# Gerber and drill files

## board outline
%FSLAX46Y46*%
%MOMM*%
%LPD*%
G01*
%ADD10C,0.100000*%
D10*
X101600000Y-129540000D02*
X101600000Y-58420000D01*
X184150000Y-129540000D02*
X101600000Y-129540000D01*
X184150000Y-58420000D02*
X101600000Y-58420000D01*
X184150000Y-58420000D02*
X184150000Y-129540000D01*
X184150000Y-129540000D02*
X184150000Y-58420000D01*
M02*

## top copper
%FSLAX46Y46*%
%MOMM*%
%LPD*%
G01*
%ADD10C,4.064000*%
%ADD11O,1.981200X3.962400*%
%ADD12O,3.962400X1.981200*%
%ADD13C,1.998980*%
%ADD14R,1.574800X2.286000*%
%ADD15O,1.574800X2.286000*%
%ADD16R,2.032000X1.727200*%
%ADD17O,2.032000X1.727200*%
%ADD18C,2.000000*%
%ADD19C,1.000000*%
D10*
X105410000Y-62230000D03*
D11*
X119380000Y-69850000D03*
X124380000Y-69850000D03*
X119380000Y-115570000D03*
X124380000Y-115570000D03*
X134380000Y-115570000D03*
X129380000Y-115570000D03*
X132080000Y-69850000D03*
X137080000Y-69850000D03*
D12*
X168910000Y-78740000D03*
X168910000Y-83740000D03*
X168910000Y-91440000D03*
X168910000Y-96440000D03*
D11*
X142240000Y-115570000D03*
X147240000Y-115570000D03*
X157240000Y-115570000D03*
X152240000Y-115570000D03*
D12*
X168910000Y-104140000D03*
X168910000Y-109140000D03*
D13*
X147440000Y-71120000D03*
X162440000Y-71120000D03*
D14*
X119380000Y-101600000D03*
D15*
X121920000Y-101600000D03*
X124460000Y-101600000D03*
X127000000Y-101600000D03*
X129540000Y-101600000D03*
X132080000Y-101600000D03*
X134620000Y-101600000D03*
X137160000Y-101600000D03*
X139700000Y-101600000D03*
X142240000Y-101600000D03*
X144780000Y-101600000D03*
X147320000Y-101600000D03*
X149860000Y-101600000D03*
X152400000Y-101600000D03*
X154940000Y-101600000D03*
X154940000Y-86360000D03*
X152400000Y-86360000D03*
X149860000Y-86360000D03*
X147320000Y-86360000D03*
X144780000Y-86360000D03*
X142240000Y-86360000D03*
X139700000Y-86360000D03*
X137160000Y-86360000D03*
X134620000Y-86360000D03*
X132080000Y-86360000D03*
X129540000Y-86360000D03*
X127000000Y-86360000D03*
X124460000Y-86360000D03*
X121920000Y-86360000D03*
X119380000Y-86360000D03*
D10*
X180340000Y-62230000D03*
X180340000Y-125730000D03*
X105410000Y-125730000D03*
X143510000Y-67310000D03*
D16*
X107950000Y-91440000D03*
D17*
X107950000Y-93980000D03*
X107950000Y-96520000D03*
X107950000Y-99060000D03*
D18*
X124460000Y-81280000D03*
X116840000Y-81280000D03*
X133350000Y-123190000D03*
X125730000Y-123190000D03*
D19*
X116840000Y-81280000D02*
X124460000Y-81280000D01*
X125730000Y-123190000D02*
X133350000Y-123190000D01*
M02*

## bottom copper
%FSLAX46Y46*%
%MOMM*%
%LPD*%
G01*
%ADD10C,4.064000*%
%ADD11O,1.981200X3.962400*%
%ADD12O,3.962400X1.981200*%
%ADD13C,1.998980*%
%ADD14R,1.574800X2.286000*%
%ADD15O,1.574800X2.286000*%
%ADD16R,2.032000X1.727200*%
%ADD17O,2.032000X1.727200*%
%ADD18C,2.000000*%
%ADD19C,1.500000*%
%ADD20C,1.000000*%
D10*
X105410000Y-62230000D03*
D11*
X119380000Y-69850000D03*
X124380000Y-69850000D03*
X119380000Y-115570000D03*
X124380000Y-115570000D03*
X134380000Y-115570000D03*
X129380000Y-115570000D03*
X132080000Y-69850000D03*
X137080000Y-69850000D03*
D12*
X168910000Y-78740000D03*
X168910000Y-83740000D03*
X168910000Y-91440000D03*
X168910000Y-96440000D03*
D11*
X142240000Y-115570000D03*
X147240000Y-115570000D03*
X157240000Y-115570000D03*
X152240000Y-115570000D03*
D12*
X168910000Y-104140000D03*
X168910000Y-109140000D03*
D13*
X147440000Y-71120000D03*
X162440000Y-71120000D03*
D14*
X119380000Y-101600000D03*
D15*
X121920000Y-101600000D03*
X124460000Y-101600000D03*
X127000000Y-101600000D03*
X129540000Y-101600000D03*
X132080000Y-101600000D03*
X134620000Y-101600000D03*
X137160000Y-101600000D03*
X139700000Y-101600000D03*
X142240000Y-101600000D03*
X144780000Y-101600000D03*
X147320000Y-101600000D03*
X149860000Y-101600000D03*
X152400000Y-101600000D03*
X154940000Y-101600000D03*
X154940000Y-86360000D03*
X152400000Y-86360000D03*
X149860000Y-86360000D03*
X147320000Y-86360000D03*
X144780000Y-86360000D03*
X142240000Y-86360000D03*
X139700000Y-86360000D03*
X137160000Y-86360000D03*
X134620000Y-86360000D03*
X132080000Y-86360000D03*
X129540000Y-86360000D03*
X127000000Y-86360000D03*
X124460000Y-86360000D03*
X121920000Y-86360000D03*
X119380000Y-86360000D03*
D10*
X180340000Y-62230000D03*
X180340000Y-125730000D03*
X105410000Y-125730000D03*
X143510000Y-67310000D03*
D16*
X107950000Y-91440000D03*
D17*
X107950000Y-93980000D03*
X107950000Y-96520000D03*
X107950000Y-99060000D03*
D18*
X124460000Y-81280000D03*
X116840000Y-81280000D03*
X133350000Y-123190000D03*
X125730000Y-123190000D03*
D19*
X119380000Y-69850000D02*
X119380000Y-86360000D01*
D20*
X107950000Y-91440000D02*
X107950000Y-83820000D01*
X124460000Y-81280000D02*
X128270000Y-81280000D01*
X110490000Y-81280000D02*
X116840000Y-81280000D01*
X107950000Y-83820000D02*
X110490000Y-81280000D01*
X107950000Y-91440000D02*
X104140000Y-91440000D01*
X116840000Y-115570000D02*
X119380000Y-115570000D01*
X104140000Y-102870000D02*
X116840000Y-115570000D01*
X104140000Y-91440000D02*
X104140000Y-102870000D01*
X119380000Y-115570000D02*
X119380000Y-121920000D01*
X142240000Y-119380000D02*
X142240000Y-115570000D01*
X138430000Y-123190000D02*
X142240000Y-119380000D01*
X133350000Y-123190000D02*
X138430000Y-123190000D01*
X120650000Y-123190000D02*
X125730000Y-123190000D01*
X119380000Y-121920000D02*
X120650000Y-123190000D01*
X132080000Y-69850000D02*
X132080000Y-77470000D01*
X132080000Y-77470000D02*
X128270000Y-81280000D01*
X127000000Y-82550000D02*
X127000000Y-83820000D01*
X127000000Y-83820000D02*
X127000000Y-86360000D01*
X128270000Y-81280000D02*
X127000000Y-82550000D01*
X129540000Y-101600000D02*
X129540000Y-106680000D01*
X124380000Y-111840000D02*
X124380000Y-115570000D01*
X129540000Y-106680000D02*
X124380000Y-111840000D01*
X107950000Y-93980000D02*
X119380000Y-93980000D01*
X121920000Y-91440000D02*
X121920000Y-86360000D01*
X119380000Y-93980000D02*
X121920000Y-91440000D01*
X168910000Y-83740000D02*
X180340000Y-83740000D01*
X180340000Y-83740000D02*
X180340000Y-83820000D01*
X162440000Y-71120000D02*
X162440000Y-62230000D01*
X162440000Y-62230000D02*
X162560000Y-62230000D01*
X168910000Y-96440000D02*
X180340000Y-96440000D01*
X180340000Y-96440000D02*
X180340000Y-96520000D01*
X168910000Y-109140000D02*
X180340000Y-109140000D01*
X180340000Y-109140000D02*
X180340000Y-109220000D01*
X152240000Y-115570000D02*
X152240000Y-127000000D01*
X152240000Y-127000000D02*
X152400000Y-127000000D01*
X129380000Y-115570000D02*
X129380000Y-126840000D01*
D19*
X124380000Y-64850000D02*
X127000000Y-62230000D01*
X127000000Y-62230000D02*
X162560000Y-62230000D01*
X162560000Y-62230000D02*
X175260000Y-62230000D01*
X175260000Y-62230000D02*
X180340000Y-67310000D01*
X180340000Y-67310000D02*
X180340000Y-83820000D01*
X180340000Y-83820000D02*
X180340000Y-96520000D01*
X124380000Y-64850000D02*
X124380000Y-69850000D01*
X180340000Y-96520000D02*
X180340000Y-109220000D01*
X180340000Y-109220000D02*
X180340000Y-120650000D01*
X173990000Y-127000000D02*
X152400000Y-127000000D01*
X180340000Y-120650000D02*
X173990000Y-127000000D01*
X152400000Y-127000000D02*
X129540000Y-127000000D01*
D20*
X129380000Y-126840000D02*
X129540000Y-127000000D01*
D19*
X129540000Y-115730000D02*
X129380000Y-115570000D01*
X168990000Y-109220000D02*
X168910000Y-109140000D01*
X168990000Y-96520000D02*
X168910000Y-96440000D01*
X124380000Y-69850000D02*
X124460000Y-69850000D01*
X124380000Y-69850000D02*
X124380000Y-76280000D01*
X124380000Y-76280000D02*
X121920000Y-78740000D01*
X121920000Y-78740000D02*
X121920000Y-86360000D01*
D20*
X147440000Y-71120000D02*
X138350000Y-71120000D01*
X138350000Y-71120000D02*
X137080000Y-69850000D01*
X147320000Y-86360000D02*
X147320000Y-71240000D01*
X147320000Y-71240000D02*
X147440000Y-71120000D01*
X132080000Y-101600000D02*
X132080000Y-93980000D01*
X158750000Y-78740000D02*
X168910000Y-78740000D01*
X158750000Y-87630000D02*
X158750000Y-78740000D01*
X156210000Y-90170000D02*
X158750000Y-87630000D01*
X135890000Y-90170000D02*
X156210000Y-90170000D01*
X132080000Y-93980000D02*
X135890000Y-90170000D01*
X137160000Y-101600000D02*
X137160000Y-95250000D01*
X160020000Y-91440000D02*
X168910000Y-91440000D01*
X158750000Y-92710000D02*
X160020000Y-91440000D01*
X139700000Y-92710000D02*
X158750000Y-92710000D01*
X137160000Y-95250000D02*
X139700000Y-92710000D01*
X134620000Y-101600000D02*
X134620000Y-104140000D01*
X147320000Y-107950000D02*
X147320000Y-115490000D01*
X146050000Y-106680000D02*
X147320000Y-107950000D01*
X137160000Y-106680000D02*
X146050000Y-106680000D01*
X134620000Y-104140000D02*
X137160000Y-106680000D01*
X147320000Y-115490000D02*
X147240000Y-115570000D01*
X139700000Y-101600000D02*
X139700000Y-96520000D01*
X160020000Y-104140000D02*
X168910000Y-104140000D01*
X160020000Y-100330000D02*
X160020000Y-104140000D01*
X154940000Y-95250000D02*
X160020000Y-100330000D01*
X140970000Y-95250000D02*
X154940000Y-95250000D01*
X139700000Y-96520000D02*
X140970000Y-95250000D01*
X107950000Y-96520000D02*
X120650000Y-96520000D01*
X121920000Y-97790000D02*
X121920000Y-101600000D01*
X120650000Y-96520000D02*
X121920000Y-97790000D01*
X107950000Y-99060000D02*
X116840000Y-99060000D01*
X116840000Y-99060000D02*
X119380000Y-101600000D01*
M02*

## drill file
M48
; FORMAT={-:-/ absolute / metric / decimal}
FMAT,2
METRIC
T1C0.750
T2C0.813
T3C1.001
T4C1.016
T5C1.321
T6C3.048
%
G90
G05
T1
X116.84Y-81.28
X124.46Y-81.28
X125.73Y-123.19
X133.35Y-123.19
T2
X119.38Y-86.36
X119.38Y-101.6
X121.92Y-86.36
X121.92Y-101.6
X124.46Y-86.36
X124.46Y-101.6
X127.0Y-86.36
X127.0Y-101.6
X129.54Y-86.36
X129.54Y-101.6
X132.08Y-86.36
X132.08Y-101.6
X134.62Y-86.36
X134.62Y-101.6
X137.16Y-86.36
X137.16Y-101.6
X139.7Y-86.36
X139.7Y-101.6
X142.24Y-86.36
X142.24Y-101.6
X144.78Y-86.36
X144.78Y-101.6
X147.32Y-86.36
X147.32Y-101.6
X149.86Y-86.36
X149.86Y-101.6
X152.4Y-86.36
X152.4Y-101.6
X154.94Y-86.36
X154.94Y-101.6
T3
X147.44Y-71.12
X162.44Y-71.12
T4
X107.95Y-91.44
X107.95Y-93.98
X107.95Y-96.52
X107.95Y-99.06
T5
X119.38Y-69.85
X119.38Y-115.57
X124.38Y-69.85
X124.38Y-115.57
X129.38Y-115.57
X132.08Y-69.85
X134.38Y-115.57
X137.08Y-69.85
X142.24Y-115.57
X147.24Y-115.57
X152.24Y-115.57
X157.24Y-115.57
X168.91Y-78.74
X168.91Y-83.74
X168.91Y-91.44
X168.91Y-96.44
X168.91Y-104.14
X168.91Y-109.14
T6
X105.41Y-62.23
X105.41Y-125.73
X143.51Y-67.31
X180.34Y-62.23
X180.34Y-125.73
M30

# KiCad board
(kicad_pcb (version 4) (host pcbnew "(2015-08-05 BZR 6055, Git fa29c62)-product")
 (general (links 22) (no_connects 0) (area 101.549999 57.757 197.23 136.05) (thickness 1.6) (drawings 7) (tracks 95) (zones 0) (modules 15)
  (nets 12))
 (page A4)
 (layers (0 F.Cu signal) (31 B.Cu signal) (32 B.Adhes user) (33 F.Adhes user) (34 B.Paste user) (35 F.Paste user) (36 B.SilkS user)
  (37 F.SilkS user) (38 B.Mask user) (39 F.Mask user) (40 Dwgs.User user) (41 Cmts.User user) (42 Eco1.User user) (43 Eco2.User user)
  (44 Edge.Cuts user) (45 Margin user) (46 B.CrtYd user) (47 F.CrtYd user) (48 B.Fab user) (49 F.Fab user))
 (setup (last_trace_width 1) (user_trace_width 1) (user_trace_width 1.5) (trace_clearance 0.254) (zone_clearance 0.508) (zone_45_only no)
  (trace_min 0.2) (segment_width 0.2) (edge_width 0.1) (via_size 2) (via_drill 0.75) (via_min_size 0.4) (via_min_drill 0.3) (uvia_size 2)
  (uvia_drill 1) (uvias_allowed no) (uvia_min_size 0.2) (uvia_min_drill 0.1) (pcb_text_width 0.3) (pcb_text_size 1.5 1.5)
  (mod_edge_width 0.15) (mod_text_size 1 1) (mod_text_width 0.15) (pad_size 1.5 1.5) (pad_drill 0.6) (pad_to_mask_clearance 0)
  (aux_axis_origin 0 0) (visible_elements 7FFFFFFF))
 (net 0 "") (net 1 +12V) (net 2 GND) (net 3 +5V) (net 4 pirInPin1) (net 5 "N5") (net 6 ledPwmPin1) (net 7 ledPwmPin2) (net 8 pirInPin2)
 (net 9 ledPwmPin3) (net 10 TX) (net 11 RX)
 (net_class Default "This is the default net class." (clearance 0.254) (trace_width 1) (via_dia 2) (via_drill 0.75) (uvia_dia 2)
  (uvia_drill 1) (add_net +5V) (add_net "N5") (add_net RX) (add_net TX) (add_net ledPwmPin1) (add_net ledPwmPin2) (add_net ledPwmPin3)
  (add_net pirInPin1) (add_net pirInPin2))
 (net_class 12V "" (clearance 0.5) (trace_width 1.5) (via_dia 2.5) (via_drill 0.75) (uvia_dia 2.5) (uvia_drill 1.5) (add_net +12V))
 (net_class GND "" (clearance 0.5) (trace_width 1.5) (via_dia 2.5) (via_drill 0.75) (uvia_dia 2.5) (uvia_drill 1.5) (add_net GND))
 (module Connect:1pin (layer F.Cu) (at 105.41 62.23)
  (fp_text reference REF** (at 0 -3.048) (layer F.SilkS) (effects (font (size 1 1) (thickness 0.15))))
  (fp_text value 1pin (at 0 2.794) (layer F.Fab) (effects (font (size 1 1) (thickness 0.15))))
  (pad 1 thru_hole circle (at 0 0) (size 4.064 4.064) (drill 3.048) (layers *.Cu *.Mask F.SilkS)))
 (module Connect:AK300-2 (layer F.Cu) (at 119.38 69.85)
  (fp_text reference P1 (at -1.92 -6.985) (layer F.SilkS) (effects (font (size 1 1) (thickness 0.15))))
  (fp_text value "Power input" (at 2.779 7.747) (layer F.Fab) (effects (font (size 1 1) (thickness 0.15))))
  (pad 1 thru_hole oval (at 0 0) (size 1.9812 3.9624) (drill 1.3208) (layers *.Cu F.Paste F.SilkS F.Mask) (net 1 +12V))
  (pad 2 thru_hole oval (at 5 0) (size 1.9812 3.9624) (drill 1.3208) (layers *.Cu F.Paste F.SilkS F.Mask) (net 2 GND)))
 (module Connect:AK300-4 (layer F.Cu) (at 119.38 115.57)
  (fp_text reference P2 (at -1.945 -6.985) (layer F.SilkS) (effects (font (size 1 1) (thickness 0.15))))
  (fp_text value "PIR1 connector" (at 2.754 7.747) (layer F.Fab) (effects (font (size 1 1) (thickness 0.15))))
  (pad 1 thru_hole oval (at 0 0) (size 1.9812 3.9624) (drill 1.3208) (layers *.Cu F.Paste F.SilkS F.Mask) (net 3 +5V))
  (pad 2 thru_hole oval (at 5 0) (size 1.9812 3.9624) (drill 1.3208) (layers *.Cu F.Paste F.SilkS F.Mask) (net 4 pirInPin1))
  (pad 4 thru_hole oval (at 15 0) (size 1.9812 3.9624) (drill 1.3208) (layers *.Cu F.Paste F.SilkS F.Mask))
  (pad 3 thru_hole oval (at 10 0) (size 1.9812 3.9624) (drill 1.3208) (layers *.Cu *.Mask F.SilkS) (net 2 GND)))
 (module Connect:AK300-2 (layer F.Cu) (at 132.08 69.85)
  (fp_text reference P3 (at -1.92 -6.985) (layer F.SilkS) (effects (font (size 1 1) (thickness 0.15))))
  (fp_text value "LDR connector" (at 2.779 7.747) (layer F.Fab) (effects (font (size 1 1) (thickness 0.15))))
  (pad 1 thru_hole oval (at 0 0) (size 1.9812 3.9624) (drill 1.3208) (layers *.Cu F.Paste F.SilkS F.Mask) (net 3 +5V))
  (pad 2 thru_hole oval (at 5 0) (size 1.9812 3.9624) (drill 1.3208) (layers *.Cu F.Paste F.SilkS F.Mask) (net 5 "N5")))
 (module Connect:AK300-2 (layer F.Cu) (at 168.91 78.74 270)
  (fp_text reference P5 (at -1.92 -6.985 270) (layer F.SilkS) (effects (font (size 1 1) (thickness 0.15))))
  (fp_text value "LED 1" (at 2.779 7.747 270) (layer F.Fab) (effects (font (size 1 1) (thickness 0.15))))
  (pad 1 thru_hole oval (at 0 0 270) (size 1.9812 3.9624) (drill 1.3208) (layers *.Cu F.Paste F.SilkS F.Mask) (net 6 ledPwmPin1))
  (pad 2 thru_hole oval (at 5 0 270) (size 1.9812 3.9624) (drill 1.3208) (layers *.Cu F.Paste F.SilkS F.Mask) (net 2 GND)))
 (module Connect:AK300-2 (layer F.Cu) (at 168.91 91.44 270)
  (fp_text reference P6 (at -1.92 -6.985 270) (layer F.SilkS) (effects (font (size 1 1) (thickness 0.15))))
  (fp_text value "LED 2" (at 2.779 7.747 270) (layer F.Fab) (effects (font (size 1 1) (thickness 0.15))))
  (pad 1 thru_hole oval (at 0 0 270) (size 1.9812 3.9624) (drill 1.3208) (layers *.Cu F.Paste F.SilkS F.Mask) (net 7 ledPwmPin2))
  (pad 2 thru_hole oval (at 5 0 270) (size 1.9812 3.9624) (drill 1.3208) (layers *.Cu F.Paste F.SilkS F.Mask) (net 2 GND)))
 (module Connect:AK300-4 (layer F.Cu) (at 142.24 115.57)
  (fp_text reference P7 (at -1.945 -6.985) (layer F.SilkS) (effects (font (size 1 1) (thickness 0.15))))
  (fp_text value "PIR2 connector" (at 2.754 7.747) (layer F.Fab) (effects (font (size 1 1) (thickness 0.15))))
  (pad 1 thru_hole oval (at 0 0) (size 1.9812 3.9624) (drill 1.3208) (layers *.Cu F.Paste F.SilkS F.Mask) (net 3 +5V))
  (pad 2 thru_hole oval (at 5 0) (size 1.9812 3.9624) (drill 1.3208) (layers *.Cu F.Paste F.SilkS F.Mask) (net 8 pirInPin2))
  (pad 4 thru_hole oval (at 15 0) (size 1.9812 3.9624) (drill 1.3208) (layers *.Cu F.Paste F.SilkS F.Mask))
  (pad 3 thru_hole oval (at 10 0) (size 1.9812 3.9624) (drill 1.3208) (layers *.Cu *.Mask F.SilkS) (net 2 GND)))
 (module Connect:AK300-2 (layer F.Cu) (at 168.91 104.14 270)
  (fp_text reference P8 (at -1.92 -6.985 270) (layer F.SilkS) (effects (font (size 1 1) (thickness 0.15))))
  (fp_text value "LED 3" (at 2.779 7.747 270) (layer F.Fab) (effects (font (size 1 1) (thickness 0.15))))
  (pad 1 thru_hole oval (at 0 0 270) (size 1.9812 3.9624) (drill 1.3208) (layers *.Cu F.Paste F.SilkS F.Mask) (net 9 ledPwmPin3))
  (pad 2 thru_hole oval (at 5 0 270) (size 1.9812 3.9624) (drill 1.3208) (layers *.Cu F.Paste F.SilkS F.Mask) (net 2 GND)))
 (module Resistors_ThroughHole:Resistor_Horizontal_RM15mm (layer F.Cu) (at 154.94 71.12)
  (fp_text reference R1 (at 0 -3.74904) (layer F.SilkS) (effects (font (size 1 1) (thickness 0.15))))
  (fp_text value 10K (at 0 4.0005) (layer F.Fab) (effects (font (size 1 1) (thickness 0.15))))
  (pad 1 thru_hole circle (at -7.5 0) (size 1.99898 1.99898) (drill 1.00076) (layers *.Cu *.SilkS *.Mask) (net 5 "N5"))
  (pad 2 thru_hole circle (at 7.5 0) (size 1.99898 1.99898) (drill 1.00076) (layers *.Cu *.SilkS *.Mask) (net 2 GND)))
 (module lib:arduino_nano (layer F.Cu) (at 138.43 93.98)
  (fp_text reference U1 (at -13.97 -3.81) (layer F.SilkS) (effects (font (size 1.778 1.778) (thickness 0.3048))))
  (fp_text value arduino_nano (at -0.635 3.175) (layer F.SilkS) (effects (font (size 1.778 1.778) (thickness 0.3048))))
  (pad TX1 thru_hole rect (at -19.05 7.62) (size 1.5748 2.286) (drill 0.8128) (layers *.Cu *.Mask F.SilkS) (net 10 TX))
  (pad RX0 thru_hole oval (at -16.51 7.62) (size 1.5748 2.286) (drill 0.8128) (layers *.Cu *.Mask F.SilkS) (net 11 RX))
  (pad RST1 thru_hole oval (at -13.97 7.62) (size 1.5748 2.286) (drill 0.8128) (layers *.Cu *.Mask F.SilkS))
  (pad GND1 thru_hole oval (at -11.43 7.62) (size 1.5748 2.286) (drill 0.8128) (layers *.Cu *.Mask F.SilkS))
  (pad D2 thru_hole oval (at -8.89 7.62) (size 1.5748 2.286) (drill 0.8128) (layers *.Cu *.Mask F.SilkS) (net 4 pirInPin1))
  (pad D3 thru_hole oval (at -6.35 7.62) (size 1.5748 2.286) (drill 0.8128) (layers *.Cu *.Mask F.SilkS) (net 6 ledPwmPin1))
  (pad D4 thru_hole oval (at -3.81 7.62) (size 1.5748 2.286) (drill 0.8128) (layers *.Cu *.Mask F.SilkS) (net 8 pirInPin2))
  (pad D5 thru_hole oval (at -1.27 7.62) (size 1.5748 2.286) (drill 0.8128) (layers *.Cu *.Mask F.SilkS) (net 7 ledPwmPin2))
  (pad D6 thru_hole oval (at 1.27 7.62) (size 1.5748 2.286) (drill 0.8128) (layers *.Cu *.Mask F.SilkS) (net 9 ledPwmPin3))
  (pad D7 thru_hole oval (at 3.81 7.62) (size 1.5748 2.286) (drill 0.8128) (layers *.Cu *.Mask F.SilkS))
  (pad D8 thru_hole oval (at 6.35 7.62) (size 1.5748 2.286) (drill 0.8128) (layers *.Cu *.Mask F.SilkS))
  (pad D9 thru_hole oval (at 8.89 7.62) (size 1.5748 2.286) (drill 0.8128) (layers *.Cu *.Mask F.SilkS))
  (pad D10 thru_hole oval (at 11.43 7.62) (size 1.5748 2.286) (drill 0.8128) (layers *.Cu *.Mask F.SilkS))
  (pad D11 thru_hole oval (at 13.97 7.62) (size 1.5748 2.286) (drill 0.8128) (layers *.Cu *.Mask F.SilkS))
  (pad D12 thru_hole oval (at 16.51 7.62) (size 1.5748 2.286) (drill 0.8128) (layers *.Cu *.Mask F.SilkS))
  (pad D13 thru_hole oval (at 16.51 -7.62) (size 1.5748 2.286) (drill 0.8128) (layers *.Cu *.Mask F.SilkS))
  (pad 3V3 thru_hole oval (at 13.97 -7.62) (size 1.5748 2.286) (drill 0.8128) (layers *.Cu *.Mask F.SilkS))
  (pad REF thru_hole oval (at 11.43 -7.62) (size 1.5748 2.286) (drill 0.8128) (layers *.Cu *.Mask F.SilkS))
  (pad A0 thru_hole oval (at 8.89 -7.62) (size 1.5748 2.286) (drill 0.8128) (layers *.Cu *.Mask F.SilkS) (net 5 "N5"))
  (pad A1 thru_hole oval (at 6.35 -7.62) (size 1.5748 2.286) (drill 0.8128) (layers *.Cu *.Mask F.SilkS))
  (pad A2 thru_hole oval (at 3.81 -7.62) (size 1.5748 2.286) (drill 0.8128) (layers *.Cu *.Mask F.SilkS))
  (pad A3 thru_hole oval (at 1.27 -7.62) (size 1.5748 2.286) (drill 0.8128) (layers *.Cu *.Mask F.SilkS))
  (pad A4 thru_hole oval (at -1.27 -7.62) (size 1.5748 2.286) (drill 0.8128) (layers *.Cu *.Mask F.SilkS))
  (pad A5 thru_hole oval (at -3.81 -7.62) (size 1.5748 2.286) (drill 0.8128) (layers *.Cu *.Mask F.SilkS))
  (pad A6 thru_hole oval (at -6.35 -7.62) (size 1.5748 2.286) (drill 0.8128) (layers *.Cu *.Mask F.SilkS))
  (pad A7 thru_hole oval (at -8.89 -7.62) (size 1.5748 2.286) (drill 0.8128) (layers *.Cu *.Mask F.SilkS))
  (pad 5V thru_hole oval (at -11.43 -7.62) (size 1.5748 2.286) (drill 0.8128) (layers *.Cu *.Mask F.SilkS) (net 3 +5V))
  (pad RST thru_hole oval (at -13.97 -7.62) (size 1.5748 2.286) (drill 0.8128) (layers *.Cu *.Mask F.SilkS))
  (pad GND thru_hole oval (at -16.51 -7.62) (size 1.5748 2.286) (drill 0.8128) (layers *.Cu *.Mask F.SilkS) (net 2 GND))
  (pad VIN thru_hole oval (at -19.05 -7.62) (size 1.5748 2.286) (drill 0.8128) (layers *.Cu *.Mask F.SilkS) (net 1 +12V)))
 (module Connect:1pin (layer F.Cu) (at 180.34 62.23)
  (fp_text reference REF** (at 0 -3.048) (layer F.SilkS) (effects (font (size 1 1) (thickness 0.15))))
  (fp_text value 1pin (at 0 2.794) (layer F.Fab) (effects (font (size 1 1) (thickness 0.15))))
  (pad 1 thru_hole circle (at 0 0) (size 4.064 4.064) (drill 3.048) (layers *.Cu *.Mask F.SilkS)))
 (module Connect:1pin (layer F.Cu) (at 180.34 125.73)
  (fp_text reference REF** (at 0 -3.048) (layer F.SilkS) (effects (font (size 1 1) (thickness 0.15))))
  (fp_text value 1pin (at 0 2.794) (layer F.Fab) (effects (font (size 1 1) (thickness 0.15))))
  (pad 1 thru_hole circle (at 0 0) (size 4.064 4.064) (drill 3.048) (layers *.Cu *.Mask F.SilkS)))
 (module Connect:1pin (layer F.Cu) (at 105.41 125.73)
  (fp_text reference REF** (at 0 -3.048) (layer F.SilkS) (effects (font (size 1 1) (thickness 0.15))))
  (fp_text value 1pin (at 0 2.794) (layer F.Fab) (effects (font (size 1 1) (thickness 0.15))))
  (pad 1 thru_hole circle (at 0 0) (size 4.064 4.064) (drill 3.048) (layers *.Cu *.Mask F.SilkS)))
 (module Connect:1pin (layer F.Cu) (at 143.51 67.31)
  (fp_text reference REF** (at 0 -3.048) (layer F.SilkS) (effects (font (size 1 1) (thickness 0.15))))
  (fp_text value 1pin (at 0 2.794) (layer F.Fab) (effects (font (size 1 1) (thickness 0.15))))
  (pad 1 thru_hole circle (at 0 0) (size 4.064 4.064) (drill 3.048) (layers *.Cu *.Mask F.SilkS)))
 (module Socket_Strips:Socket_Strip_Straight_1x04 (layer F.Cu) (at 107.95 91.44 270)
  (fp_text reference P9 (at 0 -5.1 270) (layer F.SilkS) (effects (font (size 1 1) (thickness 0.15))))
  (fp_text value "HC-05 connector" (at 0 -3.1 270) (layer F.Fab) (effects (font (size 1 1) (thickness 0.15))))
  (pad 1 thru_hole rect (at 0 0 270) (size 1.7272 2.032) (drill 1.016) (layers *.Cu *.Mask F.SilkS) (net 3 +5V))
  (pad 2 thru_hole oval (at 2.54 0 270) (size 1.7272 2.032) (drill 1.016) (layers *.Cu *.Mask F.SilkS) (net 2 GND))
  (pad 3 thru_hole oval (at 5.08 0 270) (size 1.7272 2.032) (drill 1.016) (layers *.Cu *.Mask F.SilkS) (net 11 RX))
  (pad 4 thru_hole oval (at 7.62 0 270) (size 1.7272 2.032) (drill 1.016) (layers *.Cu *.Mask F.SilkS) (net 10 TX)))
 (gr_line (start 101.6 129.54) (end 101.6 58.42) (angle 90) (layer Edge.Cuts) (width 0.1))
 (gr_line (start 184.15 129.54) (end 101.6 129.54) (angle 90) (layer Edge.Cuts) (width 0.1))
 (gr_line (start 184.15 58.42) (end 101.6 58.42) (angle 90) (layer Edge.Cuts) (width 0.1))
 (gr_line (start 184.15 58.42) (end 184.15 129.54) (angle 90) (layer Edge.Cuts) (width 0.1))
 (gr_line (start 184.15 129.54) (end 184.15 58.42) (angle 90) (layer Edge.Cuts) (width 0.1))
 (segment (start 119.38 69.85) (end 119.38 86.36) (width 1.5) (layer B.Cu) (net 1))
 (segment (start 107.95 91.44) (end 107.95 83.82) (width 1) (layer B.Cu) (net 3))
 (segment (start 124.46 81.28) (end 128.27 81.28) (width 1) (layer B.Cu) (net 3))
 (via (at 124.46 81.28) (size 2) (drill 0.75) (layers F.Cu B.Cu) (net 3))
 (segment (start 116.84 81.28) (end 124.46 81.28) (width 1) (layer F.Cu) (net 3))
 (via (at 116.84 81.28) (size 2) (drill 0.75) (layers F.Cu B.Cu) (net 3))
 (segment (start 110.49 81.28) (end 116.84 81.28) (width 1) (layer B.Cu) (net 3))
 (segment (start 107.95 83.82) (end 110.49 81.28) (width 1) (layer B.Cu) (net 3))
 (segment (start 107.95 91.44) (end 104.14 91.44) (width 1) (layer B.Cu) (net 3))
 (segment (start 116.84 115.57) (end 119.38 115.57) (width 1) (layer B.Cu) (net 3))
 (segment (start 104.14 102.87) (end 116.84 115.57) (width 1) (layer B.Cu) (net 3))
 (segment (start 104.14 91.44) (end 104.14 102.87) (width 1) (layer B.Cu) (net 3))
 (segment (start 119.38 115.57) (end 119.38 121.92) (width 1) (layer B.Cu) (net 3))
 (segment (start 142.24 119.38) (end 142.24 115.57) (width 1) (layer B.Cu) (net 3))
 (segment (start 138.43 123.19) (end 142.24 119.38) (width 1) (layer B.Cu) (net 3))
 (segment (start 133.35 123.19) (end 138.43 123.19) (width 1) (layer B.Cu) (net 3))
 (via (at 133.35 123.19) (size 2) (drill 0.75) (layers F.Cu B.Cu) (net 3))
 (segment (start 125.73 123.19) (end 133.35 123.19) (width 1) (layer F.Cu) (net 3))
 (via (at 125.73 123.19) (size 2) (drill 0.75) (layers F.Cu B.Cu) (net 3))
 (segment (start 120.65 123.19) (end 125.73 123.19) (width 1) (layer B.Cu) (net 3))
 (segment (start 119.38 121.92) (end 120.65 123.19) (width 1) (layer B.Cu) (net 3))
 (segment (start 132.08 69.85) (end 132.08 77.47) (width 1) (layer B.Cu) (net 3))
 (segment (start 132.08 77.47) (end 128.27 81.28) (width 1) (layer B.Cu) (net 3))
 (segment (start 127 82.55) (end 127 83.82) (width 1) (layer B.Cu) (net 3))
 (segment (start 127 83.82) (end 127 86.36) (width 1) (layer B.Cu) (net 3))
 (segment (start 128.27 81.28) (end 127 82.55) (width 1) (layer B.Cu) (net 3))
 (segment (start 129.54 101.6) (end 129.54 106.68) (width 1) (layer B.Cu) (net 4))
 (segment (start 124.38 111.84) (end 124.38 115.57) (width 1) (layer B.Cu) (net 4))
 (segment (start 129.54 106.68) (end 124.38 111.84) (width 1) (layer B.Cu) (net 4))
 (segment (start 107.95 93.98) (end 119.38 93.98) (width 1) (layer B.Cu) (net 2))
 (segment (start 121.92 91.44) (end 121.92 86.36) (width 1) (layer B.Cu) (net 2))
 (segment (start 119.38 93.98) (end 121.92 91.44) (width 1) (layer B.Cu) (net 2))
 (segment (start 168.91 83.74) (end 180.34 83.74) (width 1) (layer B.Cu) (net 2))
 (segment (start 180.34 83.74) (end 180.34 83.82) (width 1) (layer B.Cu) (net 2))
 (segment (start 162.44 71.12) (end 162.44 62.23) (width 1) (layer B.Cu) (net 2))
 (segment (start 162.44 62.23) (end 162.56 62.23) (width 1) (layer B.Cu) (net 2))
 (segment (start 168.91 96.44) (end 180.34 96.44) (width 1) (layer B.Cu) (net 2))
 (segment (start 180.34 96.44) (end 180.34 96.52) (width 1) (layer B.Cu) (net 2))
 (segment (start 168.91 109.14) (end 180.34 109.14) (width 1) (layer B.Cu) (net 2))
 (segment (start 180.34 109.14) (end 180.34 109.22) (width 1) (layer B.Cu) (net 2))
 (segment (start 152.24 115.57) (end 152.24 127) (width 1) (layer B.Cu) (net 2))
 (segment (start 152.24 127) (end 152.4 127) (width 1) (layer B.Cu) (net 2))
 (segment (start 129.38 115.57) (end 129.38 126.84) (width 1) (layer B.Cu) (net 2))
 (segment (start 124.38 64.85) (end 127 62.23) (width 1.5) (layer B.Cu) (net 2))
 (segment (start 127 62.23) (end 162.56 62.23) (width 1.5) (layer B.Cu) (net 2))
 (segment (start 162.56 62.23) (end 175.26 62.23) (width 1.5) (layer B.Cu) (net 2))
 (segment (start 175.26 62.23) (end 180.34 67.31) (width 1.5) (layer B.Cu) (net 2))
 (segment (start 180.34 67.31) (end 180.34 83.82) (width 1.5) (layer B.Cu) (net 2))
 (segment (start 180.34 83.82) (end 180.34 96.52) (width 1.5) (layer B.Cu) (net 2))
 (segment (start 124.38 64.85) (end 124.38 69.85) (width 1.5) (layer B.Cu) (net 2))
 (segment (start 180.34 96.52) (end 180.34 109.22) (width 1.5) (layer B.Cu) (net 2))
 (segment (start 180.34 109.22) (end 180.34 120.65) (width 1.5) (layer B.Cu) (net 2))
 (segment (start 173.99 127) (end 152.4 127) (width 1.5) (layer B.Cu) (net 2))
 (segment (start 180.34 120.65) (end 173.99 127) (width 1.5) (layer B.Cu) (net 2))
 (segment (start 152.4 127) (end 129.54 127) (width 1.5) (layer B.Cu) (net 2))
 (segment (start 129.38 126.84) (end 129.54 127) (width 1) (layer B.Cu) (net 2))
 (segment (start 129.54 115.73) (end 129.38 115.57) (width 1.5) (layer B.Cu) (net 2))
 (segment (start 168.99 109.22) (end 168.91 109.14) (width 1.5) (layer B.Cu) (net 2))
 (segment (start 168.99 96.52) (end 168.91 96.44) (width 1.5) (layer B.Cu) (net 2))
 (segment (start 124.38 69.85) (end 124.46 69.85) (width 1.5) (layer B.Cu) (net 2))
 (segment (start 124.38 69.85) (end 124.38 76.28) (width 1.5) (layer B.Cu) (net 2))
 (segment (start 124.38 76.28) (end 121.92 78.74) (width 1.5) (layer B.Cu) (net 2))
 (segment (start 121.92 78.74) (end 121.92 86.36) (width 1.5) (layer B.Cu) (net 2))
 (segment (start 147.44 71.12) (end 138.35 71.12) (width 1) (layer B.Cu) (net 5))
 (segment (start 138.35 71.12) (end 137.08 69.85) (width 1) (layer B.Cu) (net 5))
 (segment (start 147.32 86.36) (end 147.32 71.24) (width 1) (layer B.Cu) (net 5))
 (segment (start 147.32 71.24) (end 147.44 71.12) (width 1) (layer B.Cu) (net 5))
 (segment (start 132.08 101.6) (end 132.08 93.98) (width 1) (layer B.Cu) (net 6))
 (segment (start 158.75 78.74) (end 168.91 78.74) (width 1) (layer B.Cu) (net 6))
 (segment (start 158.75 87.63) (end 158.75 78.74) (width 1) (layer B.Cu) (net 6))
 (segment (start 156.21 90.17) (end 158.75 87.63) (width 1) (layer B.Cu) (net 6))
 (segment (start 135.89 90.17) (end 156.21 90.17) (width 1) (layer B.Cu) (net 6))
 (segment (start 132.08 93.98) (end 135.89 90.17) (width 1) (layer B.Cu) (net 6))
 (segment (start 137.16 101.6) (end 137.16 95.25) (width 1) (layer B.Cu) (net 7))
 (segment (start 160.02 91.44) (end 168.91 91.44) (width 1) (layer B.Cu) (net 7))
 (segment (start 158.75 92.71) (end 160.02 91.44) (width 1) (layer B.Cu) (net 7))
 (segment (start 139.7 92.71) (end 158.75 92.71) (width 1) (layer B.Cu) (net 7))
 (segment (start 137.16 95.25) (end 139.7 92.71) (width 1) (layer B.Cu) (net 7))
 (segment (start 134.62 101.6) (end 134.62 104.14) (width 1) (layer B.Cu) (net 8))
 (segment (start 147.32 107.95) (end 147.32 115.49) (width 1) (layer B.Cu) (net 8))
 (segment (start 146.05 106.68) (end 147.32 107.95) (width 1) (layer B.Cu) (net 8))
 (segment (start 137.16 106.68) (end 146.05 106.68) (width 1) (layer B.Cu) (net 8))
 (segment (start 134.62 104.14) (end 137.16 106.68) (width 1) (layer B.Cu) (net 8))
 (segment (start 147.32 115.49) (end 147.24 115.57) (width 1) (layer B.Cu) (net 8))
 (segment (start 139.7 101.6) (end 139.7 96.52) (width 1) (layer B.Cu) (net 9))
 (segment (start 160.02 104.14) (end 168.91 104.14) (width 1) (layer B.Cu) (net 9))
 (segment (start 160.02 100.33) (end 160.02 104.14) (width 1) (layer B.Cu) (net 9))
 (segment (start 154.94 95.25) (end 160.02 100.33) (width 1) (layer B.Cu) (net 9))
 (segment (start 140.97 95.25) (end 154.94 95.25) (width 1) (layer B.Cu) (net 9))
 (segment (start 139.7 96.52) (end 140.97 95.25) (width 1) (layer B.Cu) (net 9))
 (segment (start 107.95 96.52) (end 120.65 96.52) (width 1) (layer B.Cu) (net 11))
 (segment (start 121.92 97.79) (end 121.92 101.6) (width 1) (layer B.Cu) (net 11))
 (segment (start 120.65 96.52) (end 121.92 97.79) (width 1) (layer B.Cu) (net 11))
 (segment (start 107.95 99.06) (end 116.84 99.06) (width 1) (layer B.Cu) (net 10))
 (segment (start 116.84 99.06) (end 119.38 101.6) (width 1) (layer B.Cu) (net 10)))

